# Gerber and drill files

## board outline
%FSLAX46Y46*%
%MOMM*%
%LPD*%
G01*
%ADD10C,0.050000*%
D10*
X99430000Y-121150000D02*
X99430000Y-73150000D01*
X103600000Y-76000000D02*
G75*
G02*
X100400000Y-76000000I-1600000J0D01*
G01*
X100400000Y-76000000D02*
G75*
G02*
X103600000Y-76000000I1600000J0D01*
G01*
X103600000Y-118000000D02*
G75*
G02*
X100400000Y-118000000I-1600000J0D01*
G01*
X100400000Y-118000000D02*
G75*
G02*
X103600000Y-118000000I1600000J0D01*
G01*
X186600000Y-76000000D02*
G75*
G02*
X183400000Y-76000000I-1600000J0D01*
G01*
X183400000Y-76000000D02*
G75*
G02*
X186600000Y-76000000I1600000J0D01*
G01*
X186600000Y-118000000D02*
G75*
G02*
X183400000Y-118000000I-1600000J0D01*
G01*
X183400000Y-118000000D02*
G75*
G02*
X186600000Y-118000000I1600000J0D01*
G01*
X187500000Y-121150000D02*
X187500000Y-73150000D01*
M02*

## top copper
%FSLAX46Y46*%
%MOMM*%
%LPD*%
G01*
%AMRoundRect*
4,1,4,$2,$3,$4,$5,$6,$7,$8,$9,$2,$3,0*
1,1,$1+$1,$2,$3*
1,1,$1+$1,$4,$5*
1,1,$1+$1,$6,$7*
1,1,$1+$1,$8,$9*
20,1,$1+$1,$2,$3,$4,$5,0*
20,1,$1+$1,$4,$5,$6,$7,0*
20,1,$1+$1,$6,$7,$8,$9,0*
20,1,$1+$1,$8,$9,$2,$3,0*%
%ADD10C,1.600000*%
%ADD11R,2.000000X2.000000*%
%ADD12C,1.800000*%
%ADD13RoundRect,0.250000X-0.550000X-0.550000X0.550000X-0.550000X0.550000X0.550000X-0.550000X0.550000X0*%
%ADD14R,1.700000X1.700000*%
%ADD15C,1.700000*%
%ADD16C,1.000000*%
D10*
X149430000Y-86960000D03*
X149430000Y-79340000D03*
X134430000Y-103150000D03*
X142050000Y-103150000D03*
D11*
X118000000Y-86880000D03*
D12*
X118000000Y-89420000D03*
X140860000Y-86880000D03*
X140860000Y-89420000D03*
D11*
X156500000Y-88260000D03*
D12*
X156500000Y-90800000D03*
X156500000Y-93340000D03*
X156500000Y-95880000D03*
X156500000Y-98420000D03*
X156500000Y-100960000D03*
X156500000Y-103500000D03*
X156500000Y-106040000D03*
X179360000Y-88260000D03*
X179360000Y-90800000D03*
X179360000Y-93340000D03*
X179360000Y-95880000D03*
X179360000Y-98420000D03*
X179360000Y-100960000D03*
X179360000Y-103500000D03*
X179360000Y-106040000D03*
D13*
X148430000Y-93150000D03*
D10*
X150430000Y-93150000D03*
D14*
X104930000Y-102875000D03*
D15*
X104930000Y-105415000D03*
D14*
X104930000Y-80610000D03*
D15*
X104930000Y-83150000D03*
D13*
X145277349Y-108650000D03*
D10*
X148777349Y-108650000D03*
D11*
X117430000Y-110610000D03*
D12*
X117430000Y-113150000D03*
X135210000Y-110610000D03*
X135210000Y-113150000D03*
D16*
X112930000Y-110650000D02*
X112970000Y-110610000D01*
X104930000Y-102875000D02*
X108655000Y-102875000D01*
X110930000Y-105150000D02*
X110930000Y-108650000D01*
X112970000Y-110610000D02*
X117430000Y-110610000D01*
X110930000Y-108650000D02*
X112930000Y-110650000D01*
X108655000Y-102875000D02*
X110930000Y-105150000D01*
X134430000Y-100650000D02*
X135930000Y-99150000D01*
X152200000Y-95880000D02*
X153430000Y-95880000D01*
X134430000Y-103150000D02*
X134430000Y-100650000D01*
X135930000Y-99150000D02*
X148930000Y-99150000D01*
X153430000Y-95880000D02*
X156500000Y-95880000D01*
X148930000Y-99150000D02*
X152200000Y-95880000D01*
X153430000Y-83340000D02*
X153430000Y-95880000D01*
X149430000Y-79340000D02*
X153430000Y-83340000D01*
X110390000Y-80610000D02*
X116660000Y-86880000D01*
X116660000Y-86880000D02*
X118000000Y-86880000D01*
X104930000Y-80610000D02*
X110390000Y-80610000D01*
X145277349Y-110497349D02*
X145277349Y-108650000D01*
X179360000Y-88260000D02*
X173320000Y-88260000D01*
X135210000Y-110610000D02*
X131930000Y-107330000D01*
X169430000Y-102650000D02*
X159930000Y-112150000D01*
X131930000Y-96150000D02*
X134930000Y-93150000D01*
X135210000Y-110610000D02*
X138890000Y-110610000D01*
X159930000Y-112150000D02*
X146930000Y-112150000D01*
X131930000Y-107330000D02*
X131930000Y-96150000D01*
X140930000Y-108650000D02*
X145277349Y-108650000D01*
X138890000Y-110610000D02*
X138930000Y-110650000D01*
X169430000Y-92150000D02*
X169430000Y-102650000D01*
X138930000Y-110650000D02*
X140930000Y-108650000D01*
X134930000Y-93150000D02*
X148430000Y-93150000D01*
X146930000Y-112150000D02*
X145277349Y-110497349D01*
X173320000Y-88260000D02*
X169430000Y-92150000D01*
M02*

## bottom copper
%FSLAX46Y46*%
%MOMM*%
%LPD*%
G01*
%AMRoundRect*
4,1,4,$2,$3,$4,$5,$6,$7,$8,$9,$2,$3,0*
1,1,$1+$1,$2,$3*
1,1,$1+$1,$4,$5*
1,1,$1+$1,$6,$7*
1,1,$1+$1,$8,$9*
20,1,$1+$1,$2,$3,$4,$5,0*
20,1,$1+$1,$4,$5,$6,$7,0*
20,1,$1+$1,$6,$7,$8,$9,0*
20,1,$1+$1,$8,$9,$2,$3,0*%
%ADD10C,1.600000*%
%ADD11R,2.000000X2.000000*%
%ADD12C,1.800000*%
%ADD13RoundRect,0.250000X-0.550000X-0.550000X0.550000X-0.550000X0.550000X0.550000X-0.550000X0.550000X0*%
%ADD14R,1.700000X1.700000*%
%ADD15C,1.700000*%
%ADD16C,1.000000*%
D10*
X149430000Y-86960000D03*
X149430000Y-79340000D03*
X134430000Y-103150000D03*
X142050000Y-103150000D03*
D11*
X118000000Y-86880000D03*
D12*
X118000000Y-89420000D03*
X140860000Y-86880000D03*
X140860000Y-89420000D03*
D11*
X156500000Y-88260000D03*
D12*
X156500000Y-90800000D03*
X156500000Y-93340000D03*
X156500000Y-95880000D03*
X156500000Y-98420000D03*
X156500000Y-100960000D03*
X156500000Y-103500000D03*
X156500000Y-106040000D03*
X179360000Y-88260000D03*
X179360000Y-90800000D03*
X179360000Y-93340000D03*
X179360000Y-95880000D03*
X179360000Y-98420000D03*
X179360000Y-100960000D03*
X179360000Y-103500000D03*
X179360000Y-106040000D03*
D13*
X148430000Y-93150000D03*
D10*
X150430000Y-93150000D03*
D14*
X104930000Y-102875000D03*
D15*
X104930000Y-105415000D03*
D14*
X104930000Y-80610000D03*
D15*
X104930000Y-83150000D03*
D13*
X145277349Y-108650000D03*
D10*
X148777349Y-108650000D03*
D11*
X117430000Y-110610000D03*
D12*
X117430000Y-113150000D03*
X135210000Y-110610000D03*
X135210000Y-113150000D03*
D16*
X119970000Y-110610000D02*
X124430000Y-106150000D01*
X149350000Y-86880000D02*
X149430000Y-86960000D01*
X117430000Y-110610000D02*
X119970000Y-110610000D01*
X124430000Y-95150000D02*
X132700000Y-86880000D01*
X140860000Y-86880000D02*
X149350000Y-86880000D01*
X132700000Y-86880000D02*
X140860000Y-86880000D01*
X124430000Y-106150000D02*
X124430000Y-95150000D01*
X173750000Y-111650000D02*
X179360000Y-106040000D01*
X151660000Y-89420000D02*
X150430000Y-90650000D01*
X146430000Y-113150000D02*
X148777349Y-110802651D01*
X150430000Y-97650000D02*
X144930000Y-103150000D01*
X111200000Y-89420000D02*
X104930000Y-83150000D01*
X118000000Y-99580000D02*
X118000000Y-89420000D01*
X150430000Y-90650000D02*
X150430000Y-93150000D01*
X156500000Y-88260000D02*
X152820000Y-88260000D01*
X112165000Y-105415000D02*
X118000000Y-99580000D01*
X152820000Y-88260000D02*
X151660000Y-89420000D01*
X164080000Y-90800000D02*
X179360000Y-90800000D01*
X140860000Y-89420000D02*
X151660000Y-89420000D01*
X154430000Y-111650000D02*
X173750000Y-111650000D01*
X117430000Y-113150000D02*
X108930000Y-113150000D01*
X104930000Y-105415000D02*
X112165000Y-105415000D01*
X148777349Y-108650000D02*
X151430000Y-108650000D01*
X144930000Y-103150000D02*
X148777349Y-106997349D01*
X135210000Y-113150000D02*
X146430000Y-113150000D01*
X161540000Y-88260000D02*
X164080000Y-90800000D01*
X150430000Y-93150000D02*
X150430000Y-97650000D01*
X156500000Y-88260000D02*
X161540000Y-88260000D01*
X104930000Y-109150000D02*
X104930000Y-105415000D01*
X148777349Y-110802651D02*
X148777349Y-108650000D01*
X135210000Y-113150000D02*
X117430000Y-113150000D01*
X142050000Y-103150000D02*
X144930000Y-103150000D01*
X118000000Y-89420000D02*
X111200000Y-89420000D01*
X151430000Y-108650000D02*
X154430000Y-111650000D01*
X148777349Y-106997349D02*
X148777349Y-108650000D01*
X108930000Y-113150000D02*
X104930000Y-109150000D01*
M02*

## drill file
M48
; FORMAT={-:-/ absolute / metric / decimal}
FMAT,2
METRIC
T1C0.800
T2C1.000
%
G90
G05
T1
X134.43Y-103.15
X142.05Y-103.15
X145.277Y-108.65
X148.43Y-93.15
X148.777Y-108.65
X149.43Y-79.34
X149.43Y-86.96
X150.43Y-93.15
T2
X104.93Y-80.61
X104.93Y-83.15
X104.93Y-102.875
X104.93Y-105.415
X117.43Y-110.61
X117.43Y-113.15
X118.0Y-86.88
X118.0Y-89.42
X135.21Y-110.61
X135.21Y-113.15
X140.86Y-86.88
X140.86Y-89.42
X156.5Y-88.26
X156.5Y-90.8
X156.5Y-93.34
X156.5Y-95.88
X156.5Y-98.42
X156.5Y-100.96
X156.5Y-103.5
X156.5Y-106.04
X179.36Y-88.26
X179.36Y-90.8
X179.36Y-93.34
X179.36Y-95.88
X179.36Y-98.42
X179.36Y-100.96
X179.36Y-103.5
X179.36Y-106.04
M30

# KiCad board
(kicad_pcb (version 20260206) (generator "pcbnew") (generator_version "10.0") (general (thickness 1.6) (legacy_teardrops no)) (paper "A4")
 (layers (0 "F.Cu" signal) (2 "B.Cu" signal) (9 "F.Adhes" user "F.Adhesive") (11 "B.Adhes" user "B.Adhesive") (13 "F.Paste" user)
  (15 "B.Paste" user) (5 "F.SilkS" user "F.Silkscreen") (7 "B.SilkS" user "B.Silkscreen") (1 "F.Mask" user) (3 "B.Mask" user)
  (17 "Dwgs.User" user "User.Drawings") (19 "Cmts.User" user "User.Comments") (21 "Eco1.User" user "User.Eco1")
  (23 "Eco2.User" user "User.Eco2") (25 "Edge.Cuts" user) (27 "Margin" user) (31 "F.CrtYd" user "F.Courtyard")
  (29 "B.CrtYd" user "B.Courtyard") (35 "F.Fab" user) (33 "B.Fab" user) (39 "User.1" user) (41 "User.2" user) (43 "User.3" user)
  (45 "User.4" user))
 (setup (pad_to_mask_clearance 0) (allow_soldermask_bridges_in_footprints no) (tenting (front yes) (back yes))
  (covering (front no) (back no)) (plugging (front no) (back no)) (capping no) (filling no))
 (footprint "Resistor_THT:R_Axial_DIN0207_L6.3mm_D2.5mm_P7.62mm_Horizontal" (layer "F.Cu") (at 149.43 86.96 90)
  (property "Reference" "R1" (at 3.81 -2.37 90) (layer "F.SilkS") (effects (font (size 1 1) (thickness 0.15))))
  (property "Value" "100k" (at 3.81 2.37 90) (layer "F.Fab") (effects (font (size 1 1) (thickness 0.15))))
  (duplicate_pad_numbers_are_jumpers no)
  (pad "1" thru_hole circle (at 0 0 90) (size 1.6 1.6) (drill 0.8) (layers "*.Cu" "*.Mask") (remove_unused_layers no) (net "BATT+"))
  (pad "2" thru_hole circle (at 7.62 0 90) (size 1.6 1.6) (drill 0.8) (layers "*.Cu" "*.Mask") (remove_unused_layers no) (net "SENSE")))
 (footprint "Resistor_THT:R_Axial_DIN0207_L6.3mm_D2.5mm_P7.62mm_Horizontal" (layer "F.Cu") (at 134.43 103.15)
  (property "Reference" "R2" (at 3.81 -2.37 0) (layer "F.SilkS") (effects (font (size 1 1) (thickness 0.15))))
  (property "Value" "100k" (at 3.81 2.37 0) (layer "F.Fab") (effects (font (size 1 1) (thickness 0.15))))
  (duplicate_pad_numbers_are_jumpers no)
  (pad "1" thru_hole circle (at 0 0) (size 1.6 1.6) (drill 0.8) (layers "*.Cu" "*.Mask") (remove_unused_layers no) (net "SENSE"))
  (pad "2" thru_hole circle (at 7.62 0) (size 1.6 1.6) (drill 0.8) (layers "*.Cu" "*.Mask") (remove_unused_layers no) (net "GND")))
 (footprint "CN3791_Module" (layer "F.Cu") (at 129.43 88.15)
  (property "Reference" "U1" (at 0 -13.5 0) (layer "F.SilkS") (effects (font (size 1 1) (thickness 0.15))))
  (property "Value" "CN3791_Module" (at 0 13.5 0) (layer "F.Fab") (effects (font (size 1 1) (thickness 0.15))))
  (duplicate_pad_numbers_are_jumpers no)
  (pad "1" thru_hole rect (at -11.43 -1.27) (size 2 2) (drill 1) (layers "*.Cu" "*.Mask") (remove_unused_layers no) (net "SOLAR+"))
  (pad "2" thru_hole circle (at -11.43 1.27) (size 1.8 1.8) (drill 1) (layers "*.Cu" "*.Mask") (remove_unused_layers no) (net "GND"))
  (pad "3" thru_hole circle (at 11.43 -1.27) (size 1.8 1.8) (drill 1) (layers "*.Cu" "*.Mask") (remove_unused_layers no) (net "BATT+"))
  (pad "4" thru_hole circle (at 11.43 1.27) (size 1.8 1.8) (drill 1) (layers "*.Cu" "*.Mask") (remove_unused_layers no) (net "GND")))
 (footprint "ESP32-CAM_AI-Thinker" (layer "F.Cu") (at 167.93 97.15)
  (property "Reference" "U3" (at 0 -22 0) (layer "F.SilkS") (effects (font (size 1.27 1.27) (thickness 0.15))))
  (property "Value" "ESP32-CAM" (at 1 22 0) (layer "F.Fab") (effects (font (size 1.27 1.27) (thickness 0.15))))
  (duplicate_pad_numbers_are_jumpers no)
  (pad "1" thru_hole rect (at -11.43 -8.89) (size 2 2) (drill 1) (layers "*.Cu" "*.Mask") (remove_unused_layers no) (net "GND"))
  (pad "2" thru_hole circle (at -11.43 -6.35) (size 1.8 1.8) (drill 1) (layers "*.Cu" "*.Mask") (remove_unused_layers no))
  (pad "3" thru_hole circle (at -11.43 -3.81) (size 1.8 1.8) (drill 1) (layers "*.Cu" "*.Mask") (remove_unused_layers no))
  (pad "4" thru_hole circle (at -11.43 -1.27) (size 1.8 1.8) (drill 1) (layers "*.Cu" "*.Mask") (remove_unused_layers no) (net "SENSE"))
  (pad "5" thru_hole circle (at -11.43 1.27) (size 1.8 1.8) (drill 1) (layers "*.Cu" "*.Mask") (remove_unused_layers no))
  (pad "6" thru_hole circle (at -11.43 3.81) (size 1.8 1.8) (drill 1) (layers "*.Cu" "*.Mask") (remove_unused_layers no))
  (pad "7" thru_hole circle (at -11.43 6.35) (size 1.8 1.8) (drill 1) (layers "*.Cu" "*.Mask") (remove_unused_layers no))
  (pad "8" thru_hole circle (at -11.43 8.89) (size 1.8 1.8) (drill 1) (layers "*.Cu" "*.Mask") (remove_unused_layers no))
  (pad "9" thru_hole circle (at 11.43 -8.89) (size 1.8 1.8) (drill 1) (layers "*.Cu" "*.Mask") (remove_unused_layers no) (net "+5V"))
  (pad "10" thru_hole circle (at 11.43 -6.35) (size 1.8 1.8) (drill 1) (layers "*.Cu" "*.Mask") (remove_unused_layers no) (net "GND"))
  (pad "11" thru_hole circle (at 11.43 -3.81) (size 1.8 1.8) (drill 1) (layers "*.Cu" "*.Mask") (remove_unused_layers no))
  (pad "12" thru_hole circle (at 11.43 -1.27) (size 1.8 1.8) (drill 1) (layers "*.Cu" "*.Mask") (remove_unused_layers no))
  (pad "13" thru_hole circle (at 11.43 1.27) (size 1.8 1.8) (drill 1) (layers "*.Cu" "*.Mask") (remove_unused_layers no))
  (pad "14" thru_hole circle (at 11.43 3.81) (size 1.8 1.8) (drill 1) (layers "*.Cu" "*.Mask") (remove_unused_layers no))
  (pad "15" thru_hole circle (at 11.43 6.35) (size 1.8 1.8) (drill 1) (layers "*.Cu" "*.Mask") (remove_unused_layers no))
  (pad "16" thru_hole circle (at 11.43 8.89) (size 1.8 1.8) (drill 1) (layers "*.Cu" "*.Mask") (remove_unused_layers no) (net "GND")))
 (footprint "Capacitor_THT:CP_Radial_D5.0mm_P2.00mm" (layer "F.Cu") (at 148.43 93.15)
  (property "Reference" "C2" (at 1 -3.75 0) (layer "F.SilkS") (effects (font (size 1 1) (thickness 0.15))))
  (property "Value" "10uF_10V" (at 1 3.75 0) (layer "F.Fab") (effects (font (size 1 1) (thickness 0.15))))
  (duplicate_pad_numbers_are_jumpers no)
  (pad "1" thru_hole roundrect (at 0 0) (size 1.6 1.6) (drill 0.8) (layers "*.Cu" "*.Mask") (remove_unused_layers no)
   (roundrect_rratio 0.15625) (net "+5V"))
  (pad "2" thru_hole circle (at 2 0) (size 1.6 1.6) (drill 0.8) (layers "*.Cu" "*.Mask") (remove_unused_layers no) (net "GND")))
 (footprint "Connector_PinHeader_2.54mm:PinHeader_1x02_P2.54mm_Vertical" (layer "F.Cu") (at 104.93 102.875)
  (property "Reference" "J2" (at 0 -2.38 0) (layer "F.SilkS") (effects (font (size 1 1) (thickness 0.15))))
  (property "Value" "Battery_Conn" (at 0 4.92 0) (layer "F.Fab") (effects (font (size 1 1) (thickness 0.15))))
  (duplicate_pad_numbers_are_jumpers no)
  (pad "1" thru_hole rect (at 0 0) (size 1.7 1.7) (drill 1) (layers "*.Cu" "*.Mask") (remove_unused_layers no) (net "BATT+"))
  (pad "2" thru_hole circle (at 0 2.54) (size 1.7 1.7) (drill 1) (layers "*.Cu" "*.Mask") (remove_unused_layers no) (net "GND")))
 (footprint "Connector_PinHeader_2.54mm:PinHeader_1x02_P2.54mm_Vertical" (layer "F.Cu") (at 104.93 80.61)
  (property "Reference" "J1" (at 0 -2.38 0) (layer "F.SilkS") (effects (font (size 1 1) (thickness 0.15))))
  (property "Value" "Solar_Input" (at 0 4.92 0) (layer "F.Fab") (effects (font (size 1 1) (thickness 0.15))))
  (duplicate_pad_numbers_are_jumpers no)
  (pad "1" thru_hole rect (at 0 0) (size 1.7 1.7) (drill 1) (layers "*.Cu" "*.Mask") (remove_unused_layers no) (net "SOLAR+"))
  (pad "2" thru_hole circle (at 0 2.54) (size 1.7 1.7) (drill 1) (layers "*.Cu" "*.Mask") (remove_unused_layers no) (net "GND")))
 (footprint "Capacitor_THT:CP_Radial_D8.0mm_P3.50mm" (layer "F.Cu") (at 145.277349 108.65)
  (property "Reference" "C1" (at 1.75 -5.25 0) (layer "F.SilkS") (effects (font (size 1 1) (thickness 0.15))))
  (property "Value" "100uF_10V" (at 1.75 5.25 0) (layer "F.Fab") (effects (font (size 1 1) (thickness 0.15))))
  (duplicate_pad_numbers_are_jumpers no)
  (pad "1" thru_hole roundrect (at 0 0) (size 1.6 1.6) (drill 0.8) (layers "*.Cu" "*.Mask") (remove_unused_layers no)
   (roundrect_rratio 0.15625) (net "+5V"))
  (pad "2" thru_hole circle (at 3.5 0) (size 1.6 1.6) (drill 0.8) (layers "*.Cu" "*.Mask") (remove_unused_layers no) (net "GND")))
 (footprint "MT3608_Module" (layer "F.Cu") (at 126.32 111.88)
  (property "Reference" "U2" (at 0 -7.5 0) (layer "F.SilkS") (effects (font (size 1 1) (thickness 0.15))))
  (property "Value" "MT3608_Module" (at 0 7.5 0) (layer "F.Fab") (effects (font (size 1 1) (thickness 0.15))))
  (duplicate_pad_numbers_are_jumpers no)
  (pad "1" thru_hole rect (at -8.89 -1.27) (size 2 2) (drill 1) (layers "*.Cu" "*.Mask") (remove_unused_layers no) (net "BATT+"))
  (pad "2" thru_hole circle (at -8.89 1.27) (size 1.8 1.8) (drill 1) (layers "*.Cu" "*.Mask") (remove_unused_layers no) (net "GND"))
  (pad "3" thru_hole circle (at 8.89 -1.27) (size 1.8 1.8) (drill 1) (layers "*.Cu" "*.Mask") (remove_unused_layers no) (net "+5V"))
  (pad "4" thru_hole circle (at 8.89 1.27) (size 1.8 1.8) (drill 1) (layers "*.Cu" "*.Mask") (remove_unused_layers no) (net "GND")))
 (gr_line (start 99.43 121.15) (end 99.43 73.15) (stroke (width 0.05) (type default)) (layer "Edge.Cuts"))
 (gr_circle (center 102 76) (end 103.6 76) (stroke (width 0.05) (type solid)) (fill no) (layer "Edge.Cuts"))
 (gr_circle (center 102 118) (end 103.6 118) (stroke (width 0.05) (type solid)) (fill no) (layer "Edge.Cuts"))
 (gr_circle (center 185 76) (end 186.6 76) (stroke (width 0.05) (type solid)) (fill no) (layer "Edge.Cuts"))
 (gr_circle (center 185 118) (end 186.6 118) (stroke (width 0.05) (type solid)) (fill no) (layer "Edge.Cuts"))
 (gr_line (start 187.5 121.15) (end 187.5 73.15) (stroke (width 0.05) (type default)) (layer "Edge.Cuts"))
 (segment (start 112.93 110.65) (end 112.97 110.61) (width 1) (layer "F.Cu") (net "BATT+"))
 (segment (start 104.93 102.875) (end 108.655 102.875) (width 1) (layer "F.Cu") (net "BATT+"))
 (segment (start 110.93 105.15) (end 110.93 108.65) (width 1) (layer "F.Cu") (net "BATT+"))
 (segment (start 112.97 110.61) (end 117.43 110.61) (width 1) (layer "F.Cu") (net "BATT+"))
 (segment (start 110.93 108.65) (end 112.93 110.65) (width 1) (layer "F.Cu") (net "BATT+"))
 (segment (start 108.655 102.875) (end 110.93 105.15) (width 1) (layer "F.Cu") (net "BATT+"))
 (segment (start 119.97 110.61) (end 124.43 106.15) (width 1) (layer "B.Cu") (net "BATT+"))
 (segment (start 149.35 86.88) (end 149.43 86.96) (width 1) (layer "B.Cu") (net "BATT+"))
 (segment (start 117.43 110.61) (end 119.97 110.61) (width 1) (layer "B.Cu") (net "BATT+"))
 (segment (start 124.43 95.15) (end 132.7 86.88) (width 1) (layer "B.Cu") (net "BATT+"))
 (segment (start 140.86 86.88) (end 149.35 86.88) (width 1) (layer "B.Cu") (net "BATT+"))
 (segment (start 132.7 86.88) (end 140.86 86.88) (width 1) (layer "B.Cu") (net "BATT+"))
 (segment (start 124.43 106.15) (end 124.43 95.15) (width 1) (layer "B.Cu") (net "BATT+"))
 (segment (start 134.43 100.65) (end 135.93 99.15) (width 1) (layer "F.Cu") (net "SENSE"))
 (segment (start 152.2 95.88) (end 153.43 95.88) (width 1) (layer "F.Cu") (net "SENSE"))
 (segment (start 134.43 103.15) (end 134.43 100.65) (width 1) (layer "F.Cu") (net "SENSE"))
 (segment (start 135.93 99.15) (end 148.93 99.15) (width 1) (layer "F.Cu") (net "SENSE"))
 (segment (start 153.43 95.88) (end 156.5 95.88) (width 1) (layer "F.Cu") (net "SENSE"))
 (segment (start 148.93 99.15) (end 152.2 95.88) (width 1) (layer "F.Cu") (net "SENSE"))
 (segment (start 153.43 83.34) (end 153.43 95.88) (width 1) (layer "F.Cu") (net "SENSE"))
 (segment (start 149.43 79.34) (end 153.43 83.34) (width 1) (layer "F.Cu") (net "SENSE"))
 (segment (start 173.75 111.65) (end 179.36 106.04) (width 1) (layer "B.Cu") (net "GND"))
 (segment (start 151.66 89.42) (end 150.43 90.65) (width 1) (layer "B.Cu") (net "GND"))
 (segment (start 146.43 113.15) (end 148.777349 110.802651) (width 1) (layer "B.Cu") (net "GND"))
 (segment (start 150.43 97.65) (end 144.93 103.15) (width 1) (layer "B.Cu") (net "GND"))
 (segment (start 111.2 89.42) (end 104.93 83.15) (width 1) (layer "B.Cu") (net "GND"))
 (segment (start 118 99.58) (end 118 89.42) (width 1) (layer "B.Cu") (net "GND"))
 (segment (start 150.43 90.65) (end 150.43 93.15) (width 1) (layer "B.Cu") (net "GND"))
 (segment (start 156.5 88.26) (end 152.82 88.26) (width 1) (layer "B.Cu") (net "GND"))
 (segment (start 112.165 105.415) (end 118 99.58) (width 1) (layer "B.Cu") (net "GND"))
 (segment (start 152.82 88.26) (end 151.66 89.42) (width 1) (layer "B.Cu") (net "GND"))
 (segment (start 164.08 90.8) (end 179.36 90.8) (width 1) (layer "B.Cu") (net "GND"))
 (segment (start 140.86 89.42) (end 151.66 89.42) (width 1) (layer "B.Cu") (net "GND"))
 (segment (start 154.43 111.65) (end 173.75 111.65) (width 1) (layer "B.Cu") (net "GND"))
 (segment (start 117.43 113.15) (end 108.93 113.15) (width 1) (layer "B.Cu") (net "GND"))
 (segment (start 104.93 105.415) (end 112.165 105.415) (width 1) (layer "B.Cu") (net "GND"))
 (segment (start 148.777349 108.65) (end 151.43 108.65) (width 1) (layer "B.Cu") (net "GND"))
 (segment (start 144.93 103.15) (end 148.777349 106.997349) (width 1) (layer "B.Cu") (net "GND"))
 (segment (start 135.21 113.15) (end 146.43 113.15) (width 1) (layer "B.Cu") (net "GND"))
 (segment (start 161.54 88.26) (end 164.08 90.8) (width 1) (layer "B.Cu") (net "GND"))
 (segment (start 150.43 93.15) (end 150.43 97.65) (width 1) (layer "B.Cu") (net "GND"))
 (segment (start 156.5 88.26) (end 161.54 88.26) (width 1) (layer "B.Cu") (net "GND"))
 (segment (start 104.93 109.15) (end 104.93 105.415) (width 1) (layer "B.Cu") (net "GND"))
 (segment (start 148.777349 110.802651) (end 148.777349 108.65) (width 1) (layer "B.Cu") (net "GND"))
 (segment (start 135.21 113.15) (end 117.43 113.15) (width 1) (layer "B.Cu") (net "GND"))
 (segment (start 142.05 103.15) (end 144.93 103.15) (width 1) (layer "B.Cu") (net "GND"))
 (segment (start 118 89.42) (end 111.2 89.42) (width 1) (layer "B.Cu") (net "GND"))
 (segment (start 151.43 108.65) (end 154.43 111.65) (width 1) (layer "B.Cu") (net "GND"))
 (segment (start 148.777349 106.997349) (end 148.777349 108.65) (width 1) (layer "B.Cu") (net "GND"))
 (segment (start 108.93 113.15) (end 104.93 109.15) (width 1) (layer "B.Cu") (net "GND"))
 (segment (start 110.39 80.61) (end 116.66 86.88) (width 1) (layer "F.Cu") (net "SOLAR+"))
 (segment (start 116.66 86.88) (end 118 86.88) (width 1) (layer "F.Cu") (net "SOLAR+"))
 (segment (start 104.93 80.61) (end 110.39 80.61) (width 1) (layer "F.Cu") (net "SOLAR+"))
 (segment (start 145.277349 110.497349) (end 145.277349 108.65) (width 1) (layer "F.Cu") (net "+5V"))
 (segment (start 179.36 88.26) (end 173.32 88.26) (width 1) (layer "F.Cu") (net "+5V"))
 (segment (start 135.21 110.61) (end 131.93 107.33) (width 1) (layer "F.Cu") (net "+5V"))
 (segment (start 169.43 102.65) (end 159.93 112.15) (width 1) (layer "F.Cu") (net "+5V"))
 (segment (start 131.93 96.15) (end 134.93 93.15) (width 1) (layer "F.Cu") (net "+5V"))
 (segment (start 135.21 110.61) (end 138.89 110.61) (width 1) (layer "F.Cu") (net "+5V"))
 (segment (start 159.93 112.15) (end 146.93 112.15) (width 1) (layer "F.Cu") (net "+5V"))
 (segment (start 131.93 107.33) (end 131.93 96.15) (width 1) (layer "F.Cu") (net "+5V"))
 (segment (start 140.93 108.65) (end 145.277349 108.65) (width 1) (layer "F.Cu") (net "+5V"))
 (segment (start 138.89 110.61) (end 138.93 110.65) (width 1) (layer "F.Cu") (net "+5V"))
 (segment (start 169.43 92.15) (end 169.43 102.65) (width 1) (layer "F.Cu") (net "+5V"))
 (segment (start 138.93 110.65) (end 140.93 108.65) (width 1) (layer "F.Cu") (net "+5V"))
 (segment (start 134.93 93.15) (end 148.43 93.15) (width 1) (layer "F.Cu") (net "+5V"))
 (segment (start 146.93 112.15) (end 145.277349 110.497349) (width 1) (layer "F.Cu") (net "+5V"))
 (segment (start 173.32 88.26) (end 169.43 92.15) (width 1) (layer "F.Cu") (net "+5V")))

